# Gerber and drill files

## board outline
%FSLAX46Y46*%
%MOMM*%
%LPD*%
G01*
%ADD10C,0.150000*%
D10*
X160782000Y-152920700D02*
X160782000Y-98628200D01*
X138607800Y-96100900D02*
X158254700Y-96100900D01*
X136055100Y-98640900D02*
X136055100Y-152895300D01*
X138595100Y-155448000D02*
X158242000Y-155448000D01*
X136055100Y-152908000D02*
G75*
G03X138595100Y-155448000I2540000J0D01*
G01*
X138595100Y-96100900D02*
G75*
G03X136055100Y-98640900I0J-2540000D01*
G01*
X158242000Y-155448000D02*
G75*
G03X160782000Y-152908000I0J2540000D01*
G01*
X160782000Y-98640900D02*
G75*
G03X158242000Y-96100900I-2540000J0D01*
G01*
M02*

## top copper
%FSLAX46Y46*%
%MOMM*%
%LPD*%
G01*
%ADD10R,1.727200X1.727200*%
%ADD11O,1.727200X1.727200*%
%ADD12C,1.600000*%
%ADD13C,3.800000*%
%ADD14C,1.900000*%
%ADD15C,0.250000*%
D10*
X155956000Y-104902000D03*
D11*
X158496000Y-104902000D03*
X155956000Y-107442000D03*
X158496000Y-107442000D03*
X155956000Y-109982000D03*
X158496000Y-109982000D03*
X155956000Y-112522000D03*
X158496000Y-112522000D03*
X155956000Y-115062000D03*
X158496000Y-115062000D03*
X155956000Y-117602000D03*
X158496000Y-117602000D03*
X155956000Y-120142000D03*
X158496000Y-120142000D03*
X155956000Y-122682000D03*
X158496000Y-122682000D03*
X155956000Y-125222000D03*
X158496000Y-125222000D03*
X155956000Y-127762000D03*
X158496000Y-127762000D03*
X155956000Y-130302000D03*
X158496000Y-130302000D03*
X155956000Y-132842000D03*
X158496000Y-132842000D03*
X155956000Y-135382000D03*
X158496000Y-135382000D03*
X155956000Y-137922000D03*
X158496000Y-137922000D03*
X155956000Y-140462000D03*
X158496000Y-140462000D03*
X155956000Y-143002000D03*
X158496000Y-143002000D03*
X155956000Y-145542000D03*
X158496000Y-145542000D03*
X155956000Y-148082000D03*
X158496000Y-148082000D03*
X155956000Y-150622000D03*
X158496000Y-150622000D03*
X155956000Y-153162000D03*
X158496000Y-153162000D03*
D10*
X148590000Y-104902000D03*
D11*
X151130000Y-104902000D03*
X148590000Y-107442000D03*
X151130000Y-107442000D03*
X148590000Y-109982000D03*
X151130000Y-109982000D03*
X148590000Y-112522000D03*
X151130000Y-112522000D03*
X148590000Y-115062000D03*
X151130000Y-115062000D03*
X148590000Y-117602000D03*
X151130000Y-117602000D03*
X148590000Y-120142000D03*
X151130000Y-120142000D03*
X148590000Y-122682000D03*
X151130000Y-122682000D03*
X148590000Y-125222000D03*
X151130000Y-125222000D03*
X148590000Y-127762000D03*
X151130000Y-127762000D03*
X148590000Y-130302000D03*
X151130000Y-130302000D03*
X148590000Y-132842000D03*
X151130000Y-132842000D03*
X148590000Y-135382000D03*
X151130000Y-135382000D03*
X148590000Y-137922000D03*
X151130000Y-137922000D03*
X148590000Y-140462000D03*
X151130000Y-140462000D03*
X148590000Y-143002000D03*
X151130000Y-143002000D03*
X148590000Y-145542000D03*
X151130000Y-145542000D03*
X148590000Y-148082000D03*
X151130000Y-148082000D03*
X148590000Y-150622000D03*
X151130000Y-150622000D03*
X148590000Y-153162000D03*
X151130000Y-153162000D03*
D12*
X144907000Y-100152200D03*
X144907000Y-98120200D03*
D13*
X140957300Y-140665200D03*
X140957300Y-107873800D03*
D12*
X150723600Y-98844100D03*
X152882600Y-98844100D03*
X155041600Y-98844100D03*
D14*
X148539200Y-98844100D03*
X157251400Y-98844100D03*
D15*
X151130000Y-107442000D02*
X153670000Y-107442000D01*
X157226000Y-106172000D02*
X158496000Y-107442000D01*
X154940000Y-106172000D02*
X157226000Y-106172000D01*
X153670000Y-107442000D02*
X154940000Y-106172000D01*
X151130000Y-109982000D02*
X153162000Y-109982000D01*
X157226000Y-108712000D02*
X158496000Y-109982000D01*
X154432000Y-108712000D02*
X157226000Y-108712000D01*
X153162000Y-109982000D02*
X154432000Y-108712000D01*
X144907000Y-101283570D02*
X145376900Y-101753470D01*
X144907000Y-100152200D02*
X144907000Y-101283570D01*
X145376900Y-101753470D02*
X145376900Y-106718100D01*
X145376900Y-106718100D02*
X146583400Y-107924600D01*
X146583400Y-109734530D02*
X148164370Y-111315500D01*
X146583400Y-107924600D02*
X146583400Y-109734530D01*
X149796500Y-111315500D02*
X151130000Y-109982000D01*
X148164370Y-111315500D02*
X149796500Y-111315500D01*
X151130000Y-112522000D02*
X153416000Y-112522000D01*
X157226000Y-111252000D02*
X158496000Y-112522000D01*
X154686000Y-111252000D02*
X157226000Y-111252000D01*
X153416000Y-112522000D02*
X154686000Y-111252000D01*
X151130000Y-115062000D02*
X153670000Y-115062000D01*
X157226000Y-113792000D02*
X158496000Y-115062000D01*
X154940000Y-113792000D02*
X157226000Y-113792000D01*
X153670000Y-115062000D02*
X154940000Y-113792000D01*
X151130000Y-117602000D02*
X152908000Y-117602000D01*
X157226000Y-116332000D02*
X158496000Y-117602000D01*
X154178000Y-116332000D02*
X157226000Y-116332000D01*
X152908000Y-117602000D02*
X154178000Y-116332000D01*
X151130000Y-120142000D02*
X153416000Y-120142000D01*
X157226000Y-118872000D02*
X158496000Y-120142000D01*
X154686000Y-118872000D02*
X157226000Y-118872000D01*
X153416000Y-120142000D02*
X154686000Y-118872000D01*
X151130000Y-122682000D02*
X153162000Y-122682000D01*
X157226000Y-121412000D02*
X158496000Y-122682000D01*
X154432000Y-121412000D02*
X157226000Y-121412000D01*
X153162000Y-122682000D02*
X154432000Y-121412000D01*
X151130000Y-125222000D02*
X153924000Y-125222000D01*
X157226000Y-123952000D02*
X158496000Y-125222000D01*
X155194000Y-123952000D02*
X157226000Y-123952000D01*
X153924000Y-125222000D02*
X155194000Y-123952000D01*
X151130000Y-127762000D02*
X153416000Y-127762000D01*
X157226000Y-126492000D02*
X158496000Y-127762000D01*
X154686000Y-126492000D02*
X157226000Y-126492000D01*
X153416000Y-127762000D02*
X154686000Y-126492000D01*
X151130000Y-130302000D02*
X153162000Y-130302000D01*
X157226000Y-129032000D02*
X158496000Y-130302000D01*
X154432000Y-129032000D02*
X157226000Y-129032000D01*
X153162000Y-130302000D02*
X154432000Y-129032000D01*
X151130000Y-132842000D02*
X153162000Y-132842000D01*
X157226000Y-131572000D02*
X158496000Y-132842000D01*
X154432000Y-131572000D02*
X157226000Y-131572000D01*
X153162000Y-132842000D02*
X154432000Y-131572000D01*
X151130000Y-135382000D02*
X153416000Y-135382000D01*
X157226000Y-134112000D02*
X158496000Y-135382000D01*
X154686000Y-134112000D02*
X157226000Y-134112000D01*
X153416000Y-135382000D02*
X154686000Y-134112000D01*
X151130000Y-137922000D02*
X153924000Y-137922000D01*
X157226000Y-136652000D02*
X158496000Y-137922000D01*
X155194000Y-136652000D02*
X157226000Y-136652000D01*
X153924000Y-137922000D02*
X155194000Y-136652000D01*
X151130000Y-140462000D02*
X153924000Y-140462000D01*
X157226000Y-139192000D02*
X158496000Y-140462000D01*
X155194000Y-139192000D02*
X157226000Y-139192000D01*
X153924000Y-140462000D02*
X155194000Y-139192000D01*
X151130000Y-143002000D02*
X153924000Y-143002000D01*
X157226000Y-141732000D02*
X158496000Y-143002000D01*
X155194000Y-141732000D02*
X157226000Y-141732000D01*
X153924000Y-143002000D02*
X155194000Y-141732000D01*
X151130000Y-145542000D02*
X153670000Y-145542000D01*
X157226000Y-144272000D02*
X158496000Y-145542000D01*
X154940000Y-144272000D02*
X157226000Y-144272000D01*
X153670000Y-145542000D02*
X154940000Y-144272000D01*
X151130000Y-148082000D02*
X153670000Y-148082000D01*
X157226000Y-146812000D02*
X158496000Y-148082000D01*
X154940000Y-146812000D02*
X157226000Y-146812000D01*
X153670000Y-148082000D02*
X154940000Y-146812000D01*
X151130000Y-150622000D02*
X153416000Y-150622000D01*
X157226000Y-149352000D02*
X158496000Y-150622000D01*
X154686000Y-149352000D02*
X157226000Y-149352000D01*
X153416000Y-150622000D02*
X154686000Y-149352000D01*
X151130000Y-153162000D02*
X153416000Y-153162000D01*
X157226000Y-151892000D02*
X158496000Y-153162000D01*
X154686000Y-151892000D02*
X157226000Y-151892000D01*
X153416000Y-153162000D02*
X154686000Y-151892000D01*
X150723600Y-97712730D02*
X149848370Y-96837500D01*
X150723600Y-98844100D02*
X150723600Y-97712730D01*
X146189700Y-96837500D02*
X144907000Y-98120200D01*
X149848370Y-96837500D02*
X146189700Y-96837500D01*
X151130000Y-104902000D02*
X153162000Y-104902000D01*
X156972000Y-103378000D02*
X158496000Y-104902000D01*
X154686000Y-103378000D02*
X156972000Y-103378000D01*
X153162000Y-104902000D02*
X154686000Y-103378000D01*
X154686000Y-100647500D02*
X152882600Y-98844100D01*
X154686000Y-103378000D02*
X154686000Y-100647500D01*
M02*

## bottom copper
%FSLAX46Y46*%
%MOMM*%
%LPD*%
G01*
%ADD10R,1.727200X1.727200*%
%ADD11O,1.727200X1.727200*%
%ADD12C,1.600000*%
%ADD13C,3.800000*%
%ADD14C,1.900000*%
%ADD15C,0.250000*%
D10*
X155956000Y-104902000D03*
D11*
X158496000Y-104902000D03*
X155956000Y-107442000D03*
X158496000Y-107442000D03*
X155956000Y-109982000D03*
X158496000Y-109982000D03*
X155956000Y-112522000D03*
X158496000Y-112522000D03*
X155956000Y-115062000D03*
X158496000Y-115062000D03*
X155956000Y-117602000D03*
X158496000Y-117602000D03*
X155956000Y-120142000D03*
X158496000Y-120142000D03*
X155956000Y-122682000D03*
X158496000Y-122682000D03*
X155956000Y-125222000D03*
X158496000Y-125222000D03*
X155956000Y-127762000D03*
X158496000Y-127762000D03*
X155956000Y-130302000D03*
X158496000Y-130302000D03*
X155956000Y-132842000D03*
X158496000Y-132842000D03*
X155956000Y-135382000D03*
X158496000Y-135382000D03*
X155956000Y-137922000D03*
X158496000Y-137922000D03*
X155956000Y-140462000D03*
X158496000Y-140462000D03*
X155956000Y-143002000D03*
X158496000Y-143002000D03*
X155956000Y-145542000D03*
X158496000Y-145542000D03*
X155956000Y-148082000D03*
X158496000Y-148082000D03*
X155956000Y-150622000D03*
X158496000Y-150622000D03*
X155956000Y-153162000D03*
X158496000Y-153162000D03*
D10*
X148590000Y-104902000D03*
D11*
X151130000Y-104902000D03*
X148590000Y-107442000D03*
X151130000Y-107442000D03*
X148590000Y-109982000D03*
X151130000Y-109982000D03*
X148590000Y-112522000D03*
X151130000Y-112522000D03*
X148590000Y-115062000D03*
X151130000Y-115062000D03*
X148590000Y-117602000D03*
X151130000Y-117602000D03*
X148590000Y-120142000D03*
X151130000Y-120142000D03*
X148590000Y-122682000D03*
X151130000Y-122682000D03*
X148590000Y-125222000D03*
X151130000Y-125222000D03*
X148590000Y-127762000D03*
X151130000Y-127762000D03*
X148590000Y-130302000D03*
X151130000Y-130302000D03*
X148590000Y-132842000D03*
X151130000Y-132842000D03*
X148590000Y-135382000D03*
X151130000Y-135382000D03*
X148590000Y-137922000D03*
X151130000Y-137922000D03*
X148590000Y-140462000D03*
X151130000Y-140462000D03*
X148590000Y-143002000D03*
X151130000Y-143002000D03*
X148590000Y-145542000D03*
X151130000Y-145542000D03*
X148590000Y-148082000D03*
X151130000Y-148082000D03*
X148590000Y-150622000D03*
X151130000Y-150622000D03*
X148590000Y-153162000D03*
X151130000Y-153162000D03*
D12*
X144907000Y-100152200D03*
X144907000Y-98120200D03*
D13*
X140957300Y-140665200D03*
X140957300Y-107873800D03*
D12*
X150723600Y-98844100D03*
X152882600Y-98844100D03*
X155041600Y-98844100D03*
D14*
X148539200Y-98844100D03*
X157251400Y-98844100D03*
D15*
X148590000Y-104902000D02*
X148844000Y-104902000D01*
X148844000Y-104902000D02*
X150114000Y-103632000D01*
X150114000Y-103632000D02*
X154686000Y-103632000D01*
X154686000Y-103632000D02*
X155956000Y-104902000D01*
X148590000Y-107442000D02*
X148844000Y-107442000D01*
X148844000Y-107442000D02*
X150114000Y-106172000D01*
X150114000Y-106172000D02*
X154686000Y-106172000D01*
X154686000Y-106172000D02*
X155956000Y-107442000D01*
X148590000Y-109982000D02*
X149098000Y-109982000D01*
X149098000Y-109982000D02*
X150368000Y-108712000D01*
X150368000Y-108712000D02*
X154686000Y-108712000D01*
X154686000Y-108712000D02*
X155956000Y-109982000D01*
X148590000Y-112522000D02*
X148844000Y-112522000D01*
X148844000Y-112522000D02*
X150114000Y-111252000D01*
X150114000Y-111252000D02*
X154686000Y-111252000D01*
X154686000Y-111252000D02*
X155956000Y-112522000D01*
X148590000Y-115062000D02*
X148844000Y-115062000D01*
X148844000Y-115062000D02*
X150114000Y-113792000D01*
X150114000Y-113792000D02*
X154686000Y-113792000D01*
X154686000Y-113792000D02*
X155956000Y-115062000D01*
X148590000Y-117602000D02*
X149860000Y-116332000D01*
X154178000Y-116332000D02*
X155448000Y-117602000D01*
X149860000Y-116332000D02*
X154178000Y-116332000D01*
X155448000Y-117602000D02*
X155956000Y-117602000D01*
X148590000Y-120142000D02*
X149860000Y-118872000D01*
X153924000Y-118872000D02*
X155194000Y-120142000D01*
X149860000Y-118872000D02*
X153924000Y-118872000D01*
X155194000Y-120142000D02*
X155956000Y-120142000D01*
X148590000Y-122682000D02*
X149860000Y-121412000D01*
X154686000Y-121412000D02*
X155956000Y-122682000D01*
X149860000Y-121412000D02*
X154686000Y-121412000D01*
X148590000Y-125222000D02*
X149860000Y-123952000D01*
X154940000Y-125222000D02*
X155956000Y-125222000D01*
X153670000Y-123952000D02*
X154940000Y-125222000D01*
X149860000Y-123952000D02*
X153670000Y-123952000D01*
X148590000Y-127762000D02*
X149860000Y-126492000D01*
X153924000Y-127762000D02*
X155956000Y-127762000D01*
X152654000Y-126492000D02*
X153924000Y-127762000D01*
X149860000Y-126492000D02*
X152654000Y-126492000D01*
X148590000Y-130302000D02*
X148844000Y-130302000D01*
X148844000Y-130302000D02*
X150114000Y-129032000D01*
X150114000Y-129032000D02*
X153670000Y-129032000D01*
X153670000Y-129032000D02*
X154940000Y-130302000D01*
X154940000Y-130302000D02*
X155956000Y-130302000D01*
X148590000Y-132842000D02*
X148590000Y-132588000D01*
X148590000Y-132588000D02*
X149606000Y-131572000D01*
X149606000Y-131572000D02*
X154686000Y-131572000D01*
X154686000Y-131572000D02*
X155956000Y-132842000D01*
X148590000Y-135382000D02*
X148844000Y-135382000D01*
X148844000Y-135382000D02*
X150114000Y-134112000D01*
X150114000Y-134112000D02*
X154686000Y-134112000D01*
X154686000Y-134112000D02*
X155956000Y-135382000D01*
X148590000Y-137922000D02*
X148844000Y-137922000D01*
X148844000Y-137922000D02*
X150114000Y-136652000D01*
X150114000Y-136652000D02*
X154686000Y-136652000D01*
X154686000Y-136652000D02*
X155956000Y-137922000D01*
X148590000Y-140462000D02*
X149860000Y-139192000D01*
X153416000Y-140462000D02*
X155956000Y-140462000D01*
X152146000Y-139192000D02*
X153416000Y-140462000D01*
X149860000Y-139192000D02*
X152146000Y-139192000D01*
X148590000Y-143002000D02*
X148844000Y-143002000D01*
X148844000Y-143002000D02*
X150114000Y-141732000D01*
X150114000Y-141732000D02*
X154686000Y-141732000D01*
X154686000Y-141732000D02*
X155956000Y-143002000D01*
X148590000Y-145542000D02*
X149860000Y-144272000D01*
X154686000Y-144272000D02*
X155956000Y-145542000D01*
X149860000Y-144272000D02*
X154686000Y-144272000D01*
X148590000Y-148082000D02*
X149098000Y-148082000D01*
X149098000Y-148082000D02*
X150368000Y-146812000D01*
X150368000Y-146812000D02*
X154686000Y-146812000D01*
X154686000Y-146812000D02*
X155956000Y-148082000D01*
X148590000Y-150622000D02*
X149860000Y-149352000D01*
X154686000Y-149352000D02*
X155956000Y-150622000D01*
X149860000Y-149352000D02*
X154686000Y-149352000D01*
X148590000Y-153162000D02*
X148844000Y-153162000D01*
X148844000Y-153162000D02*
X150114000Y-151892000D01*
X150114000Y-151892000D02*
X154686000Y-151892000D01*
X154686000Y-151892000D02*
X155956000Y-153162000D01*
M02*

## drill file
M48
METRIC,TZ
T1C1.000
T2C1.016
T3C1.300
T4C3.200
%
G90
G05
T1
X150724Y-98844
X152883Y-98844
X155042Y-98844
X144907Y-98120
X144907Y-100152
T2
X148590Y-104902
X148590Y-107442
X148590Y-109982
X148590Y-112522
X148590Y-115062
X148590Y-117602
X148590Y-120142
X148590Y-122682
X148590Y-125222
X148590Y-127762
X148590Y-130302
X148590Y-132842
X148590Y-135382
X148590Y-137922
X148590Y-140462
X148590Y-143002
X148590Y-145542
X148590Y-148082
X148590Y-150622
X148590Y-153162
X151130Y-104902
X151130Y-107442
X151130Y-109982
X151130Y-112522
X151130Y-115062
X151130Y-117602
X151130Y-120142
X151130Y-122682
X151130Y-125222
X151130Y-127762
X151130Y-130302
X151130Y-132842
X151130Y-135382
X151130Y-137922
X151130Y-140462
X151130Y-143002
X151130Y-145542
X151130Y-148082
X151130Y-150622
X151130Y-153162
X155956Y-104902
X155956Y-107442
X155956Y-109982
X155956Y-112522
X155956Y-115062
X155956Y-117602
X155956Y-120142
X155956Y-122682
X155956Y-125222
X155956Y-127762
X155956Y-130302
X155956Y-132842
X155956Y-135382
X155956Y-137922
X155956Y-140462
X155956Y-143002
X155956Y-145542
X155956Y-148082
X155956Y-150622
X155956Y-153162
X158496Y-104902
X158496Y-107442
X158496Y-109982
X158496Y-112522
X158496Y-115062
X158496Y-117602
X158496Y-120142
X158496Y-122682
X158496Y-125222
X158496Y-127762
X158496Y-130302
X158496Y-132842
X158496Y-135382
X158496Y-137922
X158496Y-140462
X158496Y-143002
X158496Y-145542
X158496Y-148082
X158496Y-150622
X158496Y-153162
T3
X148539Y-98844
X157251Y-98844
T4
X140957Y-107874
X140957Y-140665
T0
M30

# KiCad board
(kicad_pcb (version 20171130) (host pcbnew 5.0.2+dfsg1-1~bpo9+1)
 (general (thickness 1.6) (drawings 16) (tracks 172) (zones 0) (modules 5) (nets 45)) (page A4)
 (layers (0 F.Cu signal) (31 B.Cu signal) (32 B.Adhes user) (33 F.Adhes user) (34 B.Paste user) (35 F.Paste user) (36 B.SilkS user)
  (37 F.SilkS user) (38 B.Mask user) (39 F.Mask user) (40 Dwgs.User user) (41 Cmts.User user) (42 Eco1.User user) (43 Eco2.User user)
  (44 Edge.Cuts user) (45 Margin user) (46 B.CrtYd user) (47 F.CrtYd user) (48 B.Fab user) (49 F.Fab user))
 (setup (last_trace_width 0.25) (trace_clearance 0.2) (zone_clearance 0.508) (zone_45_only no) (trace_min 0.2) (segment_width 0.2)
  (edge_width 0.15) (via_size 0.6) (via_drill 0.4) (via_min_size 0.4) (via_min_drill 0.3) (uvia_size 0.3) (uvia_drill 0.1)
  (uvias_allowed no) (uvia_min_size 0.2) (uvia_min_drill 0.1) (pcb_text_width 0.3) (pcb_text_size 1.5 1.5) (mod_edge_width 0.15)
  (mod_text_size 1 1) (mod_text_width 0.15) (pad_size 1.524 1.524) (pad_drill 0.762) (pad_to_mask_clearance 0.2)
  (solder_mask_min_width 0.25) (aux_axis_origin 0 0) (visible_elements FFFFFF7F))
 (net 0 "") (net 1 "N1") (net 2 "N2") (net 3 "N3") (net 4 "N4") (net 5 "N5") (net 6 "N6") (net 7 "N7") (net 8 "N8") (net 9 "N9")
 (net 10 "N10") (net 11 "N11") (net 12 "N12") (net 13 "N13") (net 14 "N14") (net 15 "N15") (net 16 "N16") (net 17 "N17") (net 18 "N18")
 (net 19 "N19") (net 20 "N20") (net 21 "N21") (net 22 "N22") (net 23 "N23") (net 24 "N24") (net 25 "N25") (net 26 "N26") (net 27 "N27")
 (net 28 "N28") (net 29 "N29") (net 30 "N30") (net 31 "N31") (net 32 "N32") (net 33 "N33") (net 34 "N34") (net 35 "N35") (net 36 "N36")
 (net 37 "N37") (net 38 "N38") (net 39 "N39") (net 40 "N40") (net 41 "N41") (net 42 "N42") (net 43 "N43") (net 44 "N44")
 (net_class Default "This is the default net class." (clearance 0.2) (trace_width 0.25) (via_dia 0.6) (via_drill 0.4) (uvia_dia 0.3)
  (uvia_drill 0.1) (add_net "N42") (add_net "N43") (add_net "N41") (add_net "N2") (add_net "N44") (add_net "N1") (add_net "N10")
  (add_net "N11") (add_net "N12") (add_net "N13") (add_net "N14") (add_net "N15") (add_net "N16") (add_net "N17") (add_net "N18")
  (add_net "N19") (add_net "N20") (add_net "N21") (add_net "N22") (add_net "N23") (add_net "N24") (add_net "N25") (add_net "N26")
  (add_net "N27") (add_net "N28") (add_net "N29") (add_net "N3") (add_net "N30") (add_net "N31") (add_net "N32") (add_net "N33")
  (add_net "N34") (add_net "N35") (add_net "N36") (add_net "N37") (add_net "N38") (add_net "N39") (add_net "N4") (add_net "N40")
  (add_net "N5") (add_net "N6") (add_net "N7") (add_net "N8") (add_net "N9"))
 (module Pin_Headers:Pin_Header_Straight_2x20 (layer F.Cu) (at 155.956 104.902)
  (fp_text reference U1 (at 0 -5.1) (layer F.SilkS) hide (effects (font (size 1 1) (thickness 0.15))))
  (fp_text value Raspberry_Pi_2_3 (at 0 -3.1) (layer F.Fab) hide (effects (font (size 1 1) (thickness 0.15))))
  (pad 1 thru_hole rect (at 0 0) (size 1.7272 1.7272) (drill 1.016) (layers *.Cu *.Mask) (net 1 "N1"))
  (pad 2 thru_hole oval (at 2.54 0) (size 1.7272 1.7272) (drill 1.016) (layers *.Cu *.Mask) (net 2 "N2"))
  (pad 3 thru_hole oval (at 0 2.54) (size 1.7272 1.7272) (drill 1.016) (layers *.Cu *.Mask) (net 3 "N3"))
  (pad 4 thru_hole oval (at 2.54 2.54) (size 1.7272 1.7272) (drill 1.016) (layers *.Cu *.Mask) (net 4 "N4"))
  (pad 5 thru_hole oval (at 0 5.08) (size 1.7272 1.7272) (drill 1.016) (layers *.Cu *.Mask) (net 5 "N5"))
  (pad 6 thru_hole oval (at 2.54 5.08) (size 1.7272 1.7272) (drill 1.016) (layers *.Cu *.Mask) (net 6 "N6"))
  (pad 7 thru_hole oval (at 0 7.62) (size 1.7272 1.7272) (drill 1.016) (layers *.Cu *.Mask) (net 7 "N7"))
  (pad 8 thru_hole oval (at 2.54 7.62) (size 1.7272 1.7272) (drill 1.016) (layers *.Cu *.Mask) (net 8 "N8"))
  (pad 9 thru_hole oval (at 0 10.16) (size 1.7272 1.7272) (drill 1.016) (layers *.Cu *.Mask) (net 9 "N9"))
  (pad 10 thru_hole oval (at 2.54 10.16) (size 1.7272 1.7272) (drill 1.016) (layers *.Cu *.Mask) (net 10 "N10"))
  (pad 11 thru_hole oval (at 0 12.7) (size 1.7272 1.7272) (drill 1.016) (layers *.Cu *.Mask) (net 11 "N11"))
  (pad 12 thru_hole oval (at 2.54 12.7) (size 1.7272 1.7272) (drill 1.016) (layers *.Cu *.Mask) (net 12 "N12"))
  (pad 13 thru_hole oval (at 0 15.24) (size 1.7272 1.7272) (drill 1.016) (layers *.Cu *.Mask) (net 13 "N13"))
  (pad 14 thru_hole oval (at 2.54 15.24) (size 1.7272 1.7272) (drill 1.016) (layers *.Cu *.Mask) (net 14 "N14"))
  (pad 15 thru_hole oval (at 0 17.78) (size 1.7272 1.7272) (drill 1.016) (layers *.Cu *.Mask) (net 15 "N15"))
  (pad 16 thru_hole oval (at 2.54 17.78) (size 1.7272 1.7272) (drill 1.016) (layers *.Cu *.Mask) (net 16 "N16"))
  (pad 17 thru_hole oval (at 0 20.32) (size 1.7272 1.7272) (drill 1.016) (layers *.Cu *.Mask) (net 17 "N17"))
  (pad 18 thru_hole oval (at 2.54 20.32) (size 1.7272 1.7272) (drill 1.016) (layers *.Cu *.Mask) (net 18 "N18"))
  (pad 19 thru_hole oval (at 0 22.86) (size 1.7272 1.7272) (drill 1.016) (layers *.Cu *.Mask) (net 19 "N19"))
  (pad 20 thru_hole oval (at 2.54 22.86) (size 1.7272 1.7272) (drill 1.016) (layers *.Cu *.Mask) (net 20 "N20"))
  (pad 21 thru_hole oval (at 0 25.4) (size 1.7272 1.7272) (drill 1.016) (layers *.Cu *.Mask) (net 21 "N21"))
  (pad 22 thru_hole oval (at 2.54 25.4) (size 1.7272 1.7272) (drill 1.016) (layers *.Cu *.Mask) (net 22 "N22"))
  (pad 23 thru_hole oval (at 0 27.94) (size 1.7272 1.7272) (drill 1.016) (layers *.Cu *.Mask) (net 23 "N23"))
  (pad 24 thru_hole oval (at 2.54 27.94) (size 1.7272 1.7272) (drill 1.016) (layers *.Cu *.Mask) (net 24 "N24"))
  (pad 25 thru_hole oval (at 0 30.48) (size 1.7272 1.7272) (drill 1.016) (layers *.Cu *.Mask) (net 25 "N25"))
  (pad 26 thru_hole oval (at 2.54 30.48) (size 1.7272 1.7272) (drill 1.016) (layers *.Cu *.Mask) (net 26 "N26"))
  (pad 27 thru_hole oval (at 0 33.02) (size 1.7272 1.7272) (drill 1.016) (layers *.Cu *.Mask) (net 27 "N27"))
  (pad 28 thru_hole oval (at 2.54 33.02) (size 1.7272 1.7272) (drill 1.016) (layers *.Cu *.Mask) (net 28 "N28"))
  (pad 29 thru_hole oval (at 0 35.56) (size 1.7272 1.7272) (drill 1.016) (layers *.Cu *.Mask) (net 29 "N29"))
  (pad 30 thru_hole oval (at 2.54 35.56) (size 1.7272 1.7272) (drill 1.016) (layers *.Cu *.Mask) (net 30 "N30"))
  (pad 31 thru_hole oval (at 0 38.1) (size 1.7272 1.7272) (drill 1.016) (layers *.Cu *.Mask) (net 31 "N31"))
  (pad 32 thru_hole oval (at 2.54 38.1) (size 1.7272 1.7272) (drill 1.016) (layers *.Cu *.Mask) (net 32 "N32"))
  (pad 33 thru_hole oval (at 0 40.64) (size 1.7272 1.7272) (drill 1.016) (layers *.Cu *.Mask) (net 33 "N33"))
  (pad 34 thru_hole oval (at 2.54 40.64) (size 1.7272 1.7272) (drill 1.016) (layers *.Cu *.Mask) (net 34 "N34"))
  (pad 35 thru_hole oval (at 0 43.18) (size 1.7272 1.7272) (drill 1.016) (layers *.Cu *.Mask) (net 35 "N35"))
  (pad 36 thru_hole oval (at 2.54 43.18) (size 1.7272 1.7272) (drill 1.016) (layers *.Cu *.Mask) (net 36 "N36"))
  (pad 37 thru_hole oval (at 0 45.72) (size 1.7272 1.7272) (drill 1.016) (layers *.Cu *.Mask) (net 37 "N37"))
  (pad 38 thru_hole oval (at 2.54 45.72) (size 1.7272 1.7272) (drill 1.016) (layers *.Cu *.Mask) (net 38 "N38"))
  (pad 39 thru_hole oval (at 0 48.26) (size 1.7272 1.7272) (drill 1.016) (layers *.Cu *.Mask) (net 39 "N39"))
  (pad 40 thru_hole oval (at 2.54 48.26) (size 1.7272 1.7272) (drill 1.016) (layers *.Cu *.Mask) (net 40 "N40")))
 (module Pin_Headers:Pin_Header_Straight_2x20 (layer F.Cu) (at 148.59 104.902)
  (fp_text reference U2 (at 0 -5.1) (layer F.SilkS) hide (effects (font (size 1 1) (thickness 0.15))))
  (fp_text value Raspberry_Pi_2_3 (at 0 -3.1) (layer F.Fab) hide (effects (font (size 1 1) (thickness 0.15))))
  (pad 1 thru_hole rect (at 0 0) (size 1.7272 1.7272) (drill 1.016) (layers *.Cu *.Mask) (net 1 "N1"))
  (pad 2 thru_hole oval (at 2.54 0) (size 1.7272 1.7272) (drill 1.016) (layers *.Cu *.Mask) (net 2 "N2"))
  (pad 3 thru_hole oval (at 0 2.54) (size 1.7272 1.7272) (drill 1.016) (layers *.Cu *.Mask) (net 3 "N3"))
  (pad 4 thru_hole oval (at 2.54 2.54) (size 1.7272 1.7272) (drill 1.016) (layers *.Cu *.Mask) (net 4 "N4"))
  (pad 5 thru_hole oval (at 0 5.08) (size 1.7272 1.7272) (drill 1.016) (layers *.Cu *.Mask) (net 5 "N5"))
  (pad 6 thru_hole oval (at 2.54 5.08) (size 1.7272 1.7272) (drill 1.016) (layers *.Cu *.Mask) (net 6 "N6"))
  (pad 7 thru_hole oval (at 0 7.62) (size 1.7272 1.7272) (drill 1.016) (layers *.Cu *.Mask) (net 7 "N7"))
  (pad 8 thru_hole oval (at 2.54 7.62) (size 1.7272 1.7272) (drill 1.016) (layers *.Cu *.Mask) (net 8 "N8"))
  (pad 9 thru_hole oval (at 0 10.16) (size 1.7272 1.7272) (drill 1.016) (layers *.Cu *.Mask) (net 9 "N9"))
  (pad 10 thru_hole oval (at 2.54 10.16) (size 1.7272 1.7272) (drill 1.016) (layers *.Cu *.Mask) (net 10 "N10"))
  (pad 11 thru_hole oval (at 0 12.7) (size 1.7272 1.7272) (drill 1.016) (layers *.Cu *.Mask) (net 11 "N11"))
  (pad 12 thru_hole oval (at 2.54 12.7) (size 1.7272 1.7272) (drill 1.016) (layers *.Cu *.Mask) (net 12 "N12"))
  (pad 13 thru_hole oval (at 0 15.24) (size 1.7272 1.7272) (drill 1.016) (layers *.Cu *.Mask) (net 13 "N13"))
  (pad 14 thru_hole oval (at 2.54 15.24) (size 1.7272 1.7272) (drill 1.016) (layers *.Cu *.Mask) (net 14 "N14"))
  (pad 15 thru_hole oval (at 0 17.78) (size 1.7272 1.7272) (drill 1.016) (layers *.Cu *.Mask) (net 15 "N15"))
  (pad 16 thru_hole oval (at 2.54 17.78) (size 1.7272 1.7272) (drill 1.016) (layers *.Cu *.Mask) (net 16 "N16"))
  (pad 17 thru_hole oval (at 0 20.32) (size 1.7272 1.7272) (drill 1.016) (layers *.Cu *.Mask) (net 17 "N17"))
  (pad 18 thru_hole oval (at 2.54 20.32) (size 1.7272 1.7272) (drill 1.016) (layers *.Cu *.Mask) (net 18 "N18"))
  (pad 19 thru_hole oval (at 0 22.86) (size 1.7272 1.7272) (drill 1.016) (layers *.Cu *.Mask) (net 19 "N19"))
  (pad 20 thru_hole oval (at 2.54 22.86) (size 1.7272 1.7272) (drill 1.016) (layers *.Cu *.Mask) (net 20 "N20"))
  (pad 21 thru_hole oval (at 0 25.4) (size 1.7272 1.7272) (drill 1.016) (layers *.Cu *.Mask) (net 21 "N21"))
  (pad 22 thru_hole oval (at 2.54 25.4) (size 1.7272 1.7272) (drill 1.016) (layers *.Cu *.Mask) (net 22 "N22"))
  (pad 23 thru_hole oval (at 0 27.94) (size 1.7272 1.7272) (drill 1.016) (layers *.Cu *.Mask) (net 23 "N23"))
  (pad 24 thru_hole oval (at 2.54 27.94) (size 1.7272 1.7272) (drill 1.016) (layers *.Cu *.Mask) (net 24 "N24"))
  (pad 25 thru_hole oval (at 0 30.48) (size 1.7272 1.7272) (drill 1.016) (layers *.Cu *.Mask) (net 25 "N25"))
  (pad 26 thru_hole oval (at 2.54 30.48) (size 1.7272 1.7272) (drill 1.016) (layers *.Cu *.Mask) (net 26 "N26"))
  (pad 27 thru_hole oval (at 0 33.02) (size 1.7272 1.7272) (drill 1.016) (layers *.Cu *.Mask) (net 27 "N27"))
  (pad 28 thru_hole oval (at 2.54 33.02) (size 1.7272 1.7272) (drill 1.016) (layers *.Cu *.Mask) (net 28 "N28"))
  (pad 29 thru_hole oval (at 0 35.56) (size 1.7272 1.7272) (drill 1.016) (layers *.Cu *.Mask) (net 29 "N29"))
  (pad 30 thru_hole oval (at 2.54 35.56) (size 1.7272 1.7272) (drill 1.016) (layers *.Cu *.Mask) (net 30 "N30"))
  (pad 31 thru_hole oval (at 0 38.1) (size 1.7272 1.7272) (drill 1.016) (layers *.Cu *.Mask) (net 31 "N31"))
  (pad 32 thru_hole oval (at 2.54 38.1) (size 1.7272 1.7272) (drill 1.016) (layers *.Cu *.Mask) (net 32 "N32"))
  (pad 33 thru_hole oval (at 0 40.64) (size 1.7272 1.7272) (drill 1.016) (layers *.Cu *.Mask) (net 33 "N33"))
  (pad 34 thru_hole oval (at 2.54 40.64) (size 1.7272 1.7272) (drill 1.016) (layers *.Cu *.Mask) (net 34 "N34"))
  (pad 35 thru_hole oval (at 0 43.18) (size 1.7272 1.7272) (drill 1.016) (layers *.Cu *.Mask) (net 35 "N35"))
  (pad 36 thru_hole oval (at 2.54 43.18) (size 1.7272 1.7272) (drill 1.016) (layers *.Cu *.Mask) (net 36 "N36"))
  (pad 37 thru_hole oval (at 0 45.72) (size 1.7272 1.7272) (drill 1.016) (layers *.Cu *.Mask) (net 37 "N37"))
  (pad 38 thru_hole oval (at 2.54 45.72) (size 1.7272 1.7272) (drill 1.016) (layers *.Cu *.Mask) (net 38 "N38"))
  (pad 39 thru_hole oval (at 0 48.26) (size 1.7272 1.7272) (drill 1.016) (layers *.Cu *.Mask) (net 39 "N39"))
  (pad 40 thru_hole oval (at 2.54 48.26) (size 1.7272 1.7272) (drill 1.016) (layers *.Cu *.Mask) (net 40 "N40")))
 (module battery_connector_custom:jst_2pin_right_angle (layer F.Cu) (at 144.907 99.1362 90)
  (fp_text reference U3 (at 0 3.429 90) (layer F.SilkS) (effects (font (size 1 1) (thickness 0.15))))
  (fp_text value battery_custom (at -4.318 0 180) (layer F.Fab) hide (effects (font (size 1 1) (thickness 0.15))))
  (pad 1 thru_hole circle (at -1.016 0 90) (size 1.6 1.6) (drill 1) (layers *.Cu *.Mask) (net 6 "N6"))
  (pad 2 thru_hole circle (at 1.016 0 90) (size 1.6 1.6) (drill 1) (layers *.Cu *.Mask) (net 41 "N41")))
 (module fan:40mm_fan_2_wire (layer F.Cu) (at 140.9573 124.2695 90)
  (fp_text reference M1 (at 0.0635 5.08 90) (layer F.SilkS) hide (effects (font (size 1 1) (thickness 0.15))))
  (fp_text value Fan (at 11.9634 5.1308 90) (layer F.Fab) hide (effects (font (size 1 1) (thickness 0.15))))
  (pad 1 thru_hole circle (at -16.3957 0 90) (size 3.8 3.8) (drill 3.2) (layers *.Cu *.Mask) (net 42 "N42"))
  (pad 2 thru_hole circle (at 16.3957 0 90) (size 3.8 3.8) (drill 3.2) (layers *.Cu *.Mask) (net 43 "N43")))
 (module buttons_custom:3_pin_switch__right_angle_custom (layer F.Cu) (at 152.8826 98.8441)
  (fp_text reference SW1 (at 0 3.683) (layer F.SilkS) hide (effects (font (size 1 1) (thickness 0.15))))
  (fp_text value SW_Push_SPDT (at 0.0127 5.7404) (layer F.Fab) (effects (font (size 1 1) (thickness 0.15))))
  (pad 1 thru_hole circle (at -2.159 0) (size 1.6 1.6) (drill 1) (layers *.Cu *.Mask) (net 41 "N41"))
  (pad 2 thru_hole circle (at 0 0) (size 1.6 1.6) (drill 1) (layers *.Cu *.Mask) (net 2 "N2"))
  (pad 3 thru_hole circle (at 2.159 0) (size 1.6 1.6) (drill 1) (layers *.Cu *.Mask) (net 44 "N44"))
  (pad 4 thru_hole circle (at -4.3434 0) (size 1.9 1.9) (drill 1.3) (layers *.Cu *.Mask))
  (pad 4 thru_hole circle (at 4.3688 0) (size 1.9 1.9) (drill 1.3) (layers *.Cu *.Mask)))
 (gr_line (start 160.782 152.9207) (end 160.782 98.6282) (layer Edge.Cuts) (width 0.15))
 (gr_line (start 138.6078 96.1009) (end 158.2547 96.1009) (layer Edge.Cuts) (width 0.15))
 (gr_line (start 136.0551 98.6409) (end 136.0551 152.8953) (layer Edge.Cuts) (width 0.15))
 (gr_line (start 138.5951 155.448) (end 158.242 155.448) (layer Edge.Cuts) (width 0.15))
 (gr_arc (start 138.5951 152.908) (end 138.5951 155.448) (angle 90) (layer Edge.Cuts) (width 0.15))
 (gr_arc (start 138.5951 98.6409) (end 136.0551 98.6409) (angle 90) (layer Edge.Cuts) (width 0.15))
 (gr_arc (start 158.242 152.908) (end 160.782 152.908) (angle 90) (layer Edge.Cuts) (width 0.15))
 (gr_arc (start 158.242 98.6409) (end 158.242 96.1009) (angle 90) (layer Edge.Cuts) (width 0.15))
 (segment (start 148.59 104.902) (end 148.844 104.902) (width 0.25) (layer B.Cu) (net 1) (status C00000))
 (segment (start 148.844 104.902) (end 150.114 103.632) (width 0.25) (layer B.Cu) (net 1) (status 400000))
 (segment (start 150.114 103.632) (end 154.686 103.632) (width 0.25) (layer B.Cu) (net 1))
 (segment (start 154.686 103.632) (end 155.956 104.902) (width 0.25) (layer B.Cu) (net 1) (status 800000))
 (segment (start 148.59 107.442) (end 148.844 107.442) (width 0.25) (layer B.Cu) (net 3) (status C00000))
 (segment (start 148.844 107.442) (end 150.114 106.172) (width 0.25) (layer B.Cu) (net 3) (status 400000))
 (segment (start 150.114 106.172) (end 154.686 106.172) (width 0.25) (layer B.Cu) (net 3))
 (segment (start 154.686 106.172) (end 155.956 107.442) (width 0.25) (layer B.Cu) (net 3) (status 800000))
 (segment (start 151.13 107.442) (end 153.67 107.442) (width 0.25) (layer F.Cu) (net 4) (status 400000))
 (segment (start 157.226 106.172) (end 158.496 107.442) (width 0.25) (layer F.Cu) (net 4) (status 800000))
 (segment (start 154.94 106.172) (end 157.226 106.172) (width 0.25) (layer F.Cu) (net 4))
 (segment (start 153.67 107.442) (end 154.94 106.172) (width 0.25) (layer F.Cu) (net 4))
 (segment (start 148.59 109.982) (end 149.098 109.982) (width 0.25) (layer B.Cu) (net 5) (status C00000))
 (segment (start 149.098 109.982) (end 150.368 108.712) (width 0.25) (layer B.Cu) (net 5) (status 400000))
 (segment (start 150.368 108.712) (end 154.686 108.712) (width 0.25) (layer B.Cu) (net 5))
 (segment (start 154.686 108.712) (end 155.956 109.982) (width 0.25) (layer B.Cu) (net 5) (status 800000))
 (segment (start 151.13 109.982) (end 153.162 109.982) (width 0.25) (layer F.Cu) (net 6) (status 400000))
 (segment (start 157.226 108.712) (end 158.496 109.982) (width 0.25) (layer F.Cu) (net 6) (status 800000))
 (segment (start 154.432 108.712) (end 157.226 108.712) (width 0.25) (layer F.Cu) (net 6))
 (segment (start 153.162 109.982) (end 154.432 108.712) (width 0.25) (layer F.Cu) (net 6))
 (segment (start 144.907 101.28357) (end 145.3769 101.75347) (width 0.25) (layer F.Cu) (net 6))
 (segment (start 144.907 100.1522) (end 144.907 101.28357) (width 0.25) (layer F.Cu) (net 6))
 (segment (start 145.3769 101.75347) (end 145.3769 106.7181) (width 0.25) (layer F.Cu) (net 6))
 (segment (start 145.3769 106.7181) (end 146.5834 107.9246) (width 0.25) (layer F.Cu) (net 6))
 (segment (start 146.5834 109.73453) (end 148.16437 111.3155) (width 0.25) (layer F.Cu) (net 6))
 (segment (start 146.5834 107.9246) (end 146.5834 109.73453) (width 0.25) (layer F.Cu) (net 6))
 (segment (start 149.7965 111.3155) (end 151.13 109.982) (width 0.25) (layer F.Cu) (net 6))
 (segment (start 148.16437 111.3155) (end 149.7965 111.3155) (width 0.25) (layer F.Cu) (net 6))
 (segment (start 148.59 112.522) (end 148.844 112.522) (width 0.25) (layer B.Cu) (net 7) (status C00000))
 (segment (start 148.844 112.522) (end 150.114 111.252) (width 0.25) (layer B.Cu) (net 7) (status 400000))
 (segment (start 150.114 111.252) (end 154.686 111.252) (width 0.25) (layer B.Cu) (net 7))
 (segment (start 154.686 111.252) (end 155.956 112.522) (width 0.25) (layer B.Cu) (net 7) (status 800000))
 (segment (start 151.13 112.522) (end 153.416 112.522) (width 0.25) (layer F.Cu) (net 8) (status 400000))
 (segment (start 157.226 111.252) (end 158.496 112.522) (width 0.25) (layer F.Cu) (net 8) (status 800000))
 (segment (start 154.686 111.252) (end 157.226 111.252) (width 0.25) (layer F.Cu) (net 8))
 (segment (start 153.416 112.522) (end 154.686 111.252) (width 0.25) (layer F.Cu) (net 8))
 (segment (start 148.59 115.062) (end 148.844 115.062) (width 0.25) (layer B.Cu) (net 9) (status C00000))
 (segment (start 148.844 115.062) (end 150.114 113.792) (width 0.25) (layer B.Cu) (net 9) (status 400000))
 (segment (start 150.114 113.792) (end 154.686 113.792) (width 0.25) (layer B.Cu) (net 9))
 (segment (start 154.686 113.792) (end 155.956 115.062) (width 0.25) (layer B.Cu) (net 9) (status 800000))
 (segment (start 151.13 115.062) (end 153.67 115.062) (width 0.25) (layer F.Cu) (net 10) (status 400000))
 (segment (start 157.226 113.792) (end 158.496 115.062) (width 0.25) (layer F.Cu) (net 10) (status 800000))
 (segment (start 154.94 113.792) (end 157.226 113.792) (width 0.25) (layer F.Cu) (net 10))
 (segment (start 153.67 115.062) (end 154.94 113.792) (width 0.25) (layer F.Cu) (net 10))
 (segment (start 148.59 117.602) (end 149.86 116.332) (width 0.25) (layer B.Cu) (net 11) (status 400000))
 (segment (start 154.178 116.332) (end 155.448 117.602) (width 0.25) (layer B.Cu) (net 11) (status 800000))
 (segment (start 149.86 116.332) (end 154.178 116.332) (width 0.25) (layer B.Cu) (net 11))
 (segment (start 155.448 117.602) (end 155.956 117.602) (width 0.25) (layer B.Cu) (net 11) (status C00000))
 (segment (start 151.13 117.602) (end 152.908 117.602) (width 0.25) (layer F.Cu) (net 12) (status 400000))
 (segment (start 157.226 116.332) (end 158.496 117.602) (width 0.25) (layer F.Cu) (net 12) (status 800000))
 (segment (start 154.178 116.332) (end 157.226 116.332) (width 0.25) (layer F.Cu) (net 12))
 (segment (start 152.908 117.602) (end 154.178 116.332) (width 0.25) (layer F.Cu) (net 12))
 (segment (start 148.59 120.142) (end 149.86 118.872) (width 0.25) (layer B.Cu) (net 13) (status 400000))
 (segment (start 153.924 118.872) (end 155.194 120.142) (width 0.25) (layer B.Cu) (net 13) (status 800000))
 (segment (start 149.86 118.872) (end 153.924 118.872) (width 0.25) (layer B.Cu) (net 13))
 (segment (start 155.194 120.142) (end 155.956 120.142) (width 0.25) (layer B.Cu) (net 13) (status C00000))
 (segment (start 151.13 120.142) (end 153.416 120.142) (width 0.25) (layer F.Cu) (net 14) (status 400000))
 (segment (start 157.226 118.872) (end 158.496 120.142) (width 0.25) (layer F.Cu) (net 14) (status 800000))
 (segment (start 154.686 118.872) (end 157.226 118.872) (width 0.25) (layer F.Cu) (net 14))
 (segment (start 153.416 120.142) (end 154.686 118.872) (width 0.25) (layer F.Cu) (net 14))
 (segment (start 148.59 122.682) (end 149.86 121.412) (width 0.25) (layer B.Cu) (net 15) (status 400000))
 (segment (start 154.686 121.412) (end 155.956 122.682) (width 0.25) (layer B.Cu) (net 15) (status 800000))
 (segment (start 149.86 121.412) (end 154.686 121.412) (width 0.25) (layer B.Cu) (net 15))
 (segment (start 151.13 122.682) (end 153.162 122.682) (width 0.25) (layer F.Cu) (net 16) (status 400000))
 (segment (start 157.226 121.412) (end 158.496 122.682) (width 0.25) (layer F.Cu) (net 16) (status 800000))
 (segment (start 154.432 121.412) (end 157.226 121.412) (width 0.25) (layer F.Cu) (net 16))
 (segment (start 153.162 122.682) (end 154.432 121.412) (width 0.25) (layer F.Cu) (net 16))
 (segment (start 148.59 125.222) (end 149.86 123.952) (width 0.25) (layer B.Cu) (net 17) (status 400000))
 (segment (start 154.94 125.222) (end 155.956 125.222) (width 0.25) (layer B.Cu) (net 17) (status 800000))
 (segment (start 153.67 123.952) (end 154.94 125.222) (width 0.25) (layer B.Cu) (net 17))
 (segment (start 149.86 123.952) (end 153.67 123.952) (width 0.25) (layer B.Cu) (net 17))
 (segment (start 151.13 125.222) (end 153.924 125.222) (width 0.25) (layer F.Cu) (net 18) (status 400000))
 (segment (start 157.226 123.952) (end 158.496 125.222) (width 0.25) (layer F.Cu) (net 18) (status 800000))
 (segment (start 155.194 123.952) (end 157.226 123.952) (width 0.25) (layer F.Cu) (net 18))
 (segment (start 153.924 125.222) (end 155.194 123.952) (width 0.25) (layer F.Cu) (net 18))
 (segment (start 148.59 127.762) (end 149.86 126.492) (width 0.25) (layer B.Cu) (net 19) (status 400000))
 (segment (start 153.924 127.762) (end 155.956 127.762) (width 0.25) (layer B.Cu) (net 19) (status 800000))
 (segment (start 152.654 126.492) (end 153.924 127.762) (width 0.25) (layer B.Cu) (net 19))
 (segment (start 149.86 126.492) (end 152.654 126.492) (width 0.25) (layer B.Cu) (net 19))
 (segment (start 151.13 127.762) (end 153.416 127.762) (width 0.25) (layer F.Cu) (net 20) (status 400000))
 (segment (start 157.226 126.492) (end 158.496 127.762) (width 0.25) (layer F.Cu) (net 20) (status 800000))
 (segment (start 154.686 126.492) (end 157.226 126.492) (width 0.25) (layer F.Cu) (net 20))
 (segment (start 153.416 127.762) (end 154.686 126.492) (width 0.25) (layer F.Cu) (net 20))
 (segment (start 148.59 130.302) (end 148.844 130.302) (width 0.25) (layer B.Cu) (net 21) (status C00000))
 (segment (start 148.844 130.302) (end 150.114 129.032) (width 0.25) (layer B.Cu) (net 21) (status 400000))
 (segment (start 150.114 129.032) (end 153.67 129.032) (width 0.25) (layer B.Cu) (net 21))
 (segment (start 153.67 129.032) (end 154.94 130.302) (width 0.25) (layer B.Cu) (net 21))
 (segment (start 154.94 130.302) (end 155.956 130.302) (width 0.25) (layer B.Cu) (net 21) (status 800000))
 (segment (start 151.13 130.302) (end 153.162 130.302) (width 0.25) (layer F.Cu) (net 22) (status 400000))
 (segment (start 157.226 129.032) (end 158.496 130.302) (width 0.25) (layer F.Cu) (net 22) (status 800000))
 (segment (start 154.432 129.032) (end 157.226 129.032) (width 0.25) (layer F.Cu) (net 22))
 (segment (start 153.162 130.302) (end 154.432 129.032) (width 0.25) (layer F.Cu) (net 22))
 (segment (start 148.59 132.842) (end 148.59 132.588) (width 0.25) (layer B.Cu) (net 23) (status C00000))
 (segment (start 148.59 132.588) (end 149.606 131.572) (width 0.25) (layer B.Cu) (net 23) (status 400000))
 (segment (start 149.606 131.572) (end 154.686 131.572) (width 0.25) (layer B.Cu) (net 23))
 (segment (start 154.686 131.572) (end 155.956 132.842) (width 0.25) (layer B.Cu) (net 23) (status 800000))
 (segment (start 151.13 132.842) (end 153.162 132.842) (width 0.25) (layer F.Cu) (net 24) (status 400000))
 (segment (start 157.226 131.572) (end 158.496 132.842) (width 0.25) (layer F.Cu) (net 24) (status 800000))
 (segment (start 154.432 131.572) (end 157.226 131.572) (width 0.25) (layer F.Cu) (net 24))
 (segment (start 153.162 132.842) (end 154.432 131.572) (width 0.25) (layer F.Cu) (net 24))
 (segment (start 148.59 135.382) (end 148.844 135.382) (width 0.25) (layer B.Cu) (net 25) (status C00000))
 (segment (start 148.844 135.382) (end 150.114 134.112) (width 0.25) (layer B.Cu) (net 25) (status 400000))
 (segment (start 150.114 134.112) (end 154.686 134.112) (width 0.25) (layer B.Cu) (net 25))
 (segment (start 154.686 134.112) (end 155.956 135.382) (width 0.25) (layer B.Cu) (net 25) (status 800000))
 (segment (start 151.13 135.382) (end 153.416 135.382) (width 0.25) (layer F.Cu) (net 26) (status 400000))
 (segment (start 157.226 134.112) (end 158.496 135.382) (width 0.25) (layer F.Cu) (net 26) (status 800000))
 (segment (start 154.686 134.112) (end 157.226 134.112) (width 0.25) (layer F.Cu) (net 26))
 (segment (start 153.416 135.382) (end 154.686 134.112) (width 0.25) (layer F.Cu) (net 26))
 (segment (start 148.59 137.922) (end 148.844 137.922) (width 0.25) (layer B.Cu) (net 27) (status C00000))
 (segment (start 148.844 137.922) (end 150.114 136.652) (width 0.25) (layer B.Cu) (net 27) (status 400000))
 (segment (start 150.114 136.652) (end 154.686 136.652) (width 0.25) (layer B.Cu) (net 27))
 (segment (start 154.686 136.652) (end 155.956 137.922) (width 0.25) (layer B.Cu) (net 27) (status 800000))
 (segment (start 151.13 137.922) (end 153.924 137.922) (width 0.25) (layer F.Cu) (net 28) (status 400000))
 (segment (start 157.226 136.652) (end 158.496 137.922) (width 0.25) (layer F.Cu) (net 28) (status 800000))
 (segment (start 155.194 136.652) (end 157.226 136.652) (width 0.25) (layer F.Cu) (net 28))
 (segment (start 153.924 137.922) (end 155.194 136.652) (width 0.25) (layer F.Cu) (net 28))
 (segment (start 148.59 140.462) (end 149.86 139.192) (width 0.25) (layer B.Cu) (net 29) (status 400000))
 (segment (start 153.416 140.462) (end 155.956 140.462) (width 0.25) (layer B.Cu) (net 29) (status 800000))
 (segment (start 152.146 139.192) (end 153.416 140.462) (width 0.25) (layer B.Cu) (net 29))
 (segment (start 149.86 139.192) (end 152.146 139.192) (width 0.25) (layer B.Cu) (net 29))
 (segment (start 151.13 140.462) (end 153.924 140.462) (width 0.25) (layer F.Cu) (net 30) (status 400000))
 (segment (start 157.226 139.192) (end 158.496 140.462) (width 0.25) (layer F.Cu) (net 30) (status 800000))
 (segment (start 155.194 139.192) (end 157.226 139.192) (width 0.25) (layer F.Cu) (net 30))
 (segment (start 153.924 140.462) (end 155.194 139.192) (width 0.25) (layer F.Cu) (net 30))
 (segment (start 148.59 143.002) (end 148.844 143.002) (width 0.25) (layer B.Cu) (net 31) (status C00000))
 (segment (start 148.844 143.002) (end 150.114 141.732) (width 0.25) (layer B.Cu) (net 31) (status 400000))
 (segment (start 150.114 141.732) (end 154.686 141.732) (width 0.25) (layer B.Cu) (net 31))
 (segment (start 154.686 141.732) (end 155.956 143.002) (width 0.25) (layer B.Cu) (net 31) (status 800000))
 (segment (start 151.13 143.002) (end 153.924 143.002) (width 0.25) (layer F.Cu) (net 32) (status 400000))
 (segment (start 157.226 141.732) (end 158.496 143.002) (width 0.25) (layer F.Cu) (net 32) (status 800000))
 (segment (start 155.194 141.732) (end 157.226 141.732) (width 0.25) (layer F.Cu) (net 32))
 (segment (start 153.924 143.002) (end 155.194 141.732) (width 0.25) (layer F.Cu) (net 32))
 (segment (start 148.59 145.542) (end 149.86 144.272) (width 0.25) (layer B.Cu) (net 33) (status 400000))
 (segment (start 154.686 144.272) (end 155.956 145.542) (width 0.25) (layer B.Cu) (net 33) (status 800000))
 (segment (start 149.86 144.272) (end 154.686 144.272) (width 0.25) (layer B.Cu) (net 33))
 (segment (start 151.13 145.542) (end 153.67 145.542) (width 0.25) (layer F.Cu) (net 34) (status 400000))
 (segment (start 157.226 144.272) (end 158.496 145.542) (width 0.25) (layer F.Cu) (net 34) (status 800000))
 (segment (start 154.94 144.272) (end 157.226 144.272) (width 0.25) (layer F.Cu) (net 34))
 (segment (start 153.67 145.542) (end 154.94 144.272) (width 0.25) (layer F.Cu) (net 34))
 (segment (start 148.59 148.082) (end 149.098 148.082) (width 0.25) (layer B.Cu) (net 35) (status C00000))
 (segment (start 149.098 148.082) (end 150.368 146.812) (width 0.25) (layer B.Cu) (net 35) (status 400000))
 (segment (start 150.368 146.812) (end 154.686 146.812) (width 0.25) (layer B.Cu) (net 35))
 (segment (start 154.686 146.812) (end 155.956 148.082) (width 0.25) (layer B.Cu) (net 35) (status 800000))
 (segment (start 151.13 148.082) (end 153.67 148.082) (width 0.25) (layer F.Cu) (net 36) (status 400000))
 (segment (start 157.226 146.812) (end 158.496 148.082) (width 0.25) (layer F.Cu) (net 36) (status 800000))
 (segment (start 154.94 146.812) (end 157.226 146.812) (width 0.25) (layer F.Cu) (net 36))
 (segment (start 153.67 148.082) (end 154.94 146.812) (width 0.25) (layer F.Cu) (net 36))
 (segment (start 148.59 150.622) (end 149.86 149.352) (width 0.25) (layer B.Cu) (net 37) (status 400000))
 (segment (start 154.686 149.352) (end 155.956 150.622) (width 0.25) (layer B.Cu) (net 37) (status 800000))
 (segment (start 149.86 149.352) (end 154.686 149.352) (width 0.25) (layer B.Cu) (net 37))
 (segment (start 151.13 150.622) (end 153.416 150.622) (width 0.25) (layer F.Cu) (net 38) (status 400000))
 (segment (start 157.226 149.352) (end 158.496 150.622) (width 0.25) (layer F.Cu) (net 38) (status 800000))
 (segment (start 154.686 149.352) (end 157.226 149.352) (width 0.25) (layer F.Cu) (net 38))
 (segment (start 153.416 150.622) (end 154.686 149.352) (width 0.25) (layer F.Cu) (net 38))
 (segment (start 148.59 153.162) (end 148.844 153.162) (width 0.25) (layer B.Cu) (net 39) (status C00000))
 (segment (start 148.844 153.162) (end 150.114 151.892) (width 0.25) (layer B.Cu) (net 39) (status 400000))
 (segment (start 150.114 151.892) (end 154.686 151.892) (width 0.25) (layer B.Cu) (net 39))
 (segment (start 154.686 151.892) (end 155.956 153.162) (width 0.25) (layer B.Cu) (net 39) (status 800000))
 (segment (start 151.13 153.162) (end 153.416 153.162) (width 0.25) (layer F.Cu) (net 40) (status 400000))
 (segment (start 157.226 151.892) (end 158.496 153.162) (width 0.25) (layer F.Cu) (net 40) (status 800000))
 (segment (start 154.686 151.892) (end 157.226 151.892) (width 0.25) (layer F.Cu) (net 40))
 (segment (start 153.416 153.162) (end 154.686 151.892) (width 0.25) (layer F.Cu) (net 40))
 (segment (start 150.7236 97.71273) (end 149.84837 96.8375) (width 0.25) (layer F.Cu) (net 41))
 (segment (start 150.7236 98.8441) (end 150.7236 97.71273) (width 0.25) (layer F.Cu) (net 41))
 (segment (start 146.1897 96.8375) (end 144.907 98.1202) (width 0.25) (layer F.Cu) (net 41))
 (segment (start 149.84837 96.8375) (end 146.1897 96.8375) (width 0.25) (layer F.Cu) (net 41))
 (segment (start 151.13 104.902) (end 153.162 104.902) (width 0.25) (layer F.Cu) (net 2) (status 400000))
 (segment (start 156.972 103.378) (end 158.496 104.902) (width 0.25) (layer F.Cu) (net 2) (status 800000))
 (segment (start 154.686 103.378) (end 156.972 103.378) (width 0.25) (layer F.Cu) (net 2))
 (segment (start 153.162 104.902) (end 154.686 103.378) (width 0.25) (layer F.Cu) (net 2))
 (segment (start 154.686 100.6475) (end 152.8826 98.8441) (width 0.25) (layer F.Cu) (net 2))
 (segment (start 154.686 103.378) (end 154.686 100.6475) (width 0.25) (layer F.Cu) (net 2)))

